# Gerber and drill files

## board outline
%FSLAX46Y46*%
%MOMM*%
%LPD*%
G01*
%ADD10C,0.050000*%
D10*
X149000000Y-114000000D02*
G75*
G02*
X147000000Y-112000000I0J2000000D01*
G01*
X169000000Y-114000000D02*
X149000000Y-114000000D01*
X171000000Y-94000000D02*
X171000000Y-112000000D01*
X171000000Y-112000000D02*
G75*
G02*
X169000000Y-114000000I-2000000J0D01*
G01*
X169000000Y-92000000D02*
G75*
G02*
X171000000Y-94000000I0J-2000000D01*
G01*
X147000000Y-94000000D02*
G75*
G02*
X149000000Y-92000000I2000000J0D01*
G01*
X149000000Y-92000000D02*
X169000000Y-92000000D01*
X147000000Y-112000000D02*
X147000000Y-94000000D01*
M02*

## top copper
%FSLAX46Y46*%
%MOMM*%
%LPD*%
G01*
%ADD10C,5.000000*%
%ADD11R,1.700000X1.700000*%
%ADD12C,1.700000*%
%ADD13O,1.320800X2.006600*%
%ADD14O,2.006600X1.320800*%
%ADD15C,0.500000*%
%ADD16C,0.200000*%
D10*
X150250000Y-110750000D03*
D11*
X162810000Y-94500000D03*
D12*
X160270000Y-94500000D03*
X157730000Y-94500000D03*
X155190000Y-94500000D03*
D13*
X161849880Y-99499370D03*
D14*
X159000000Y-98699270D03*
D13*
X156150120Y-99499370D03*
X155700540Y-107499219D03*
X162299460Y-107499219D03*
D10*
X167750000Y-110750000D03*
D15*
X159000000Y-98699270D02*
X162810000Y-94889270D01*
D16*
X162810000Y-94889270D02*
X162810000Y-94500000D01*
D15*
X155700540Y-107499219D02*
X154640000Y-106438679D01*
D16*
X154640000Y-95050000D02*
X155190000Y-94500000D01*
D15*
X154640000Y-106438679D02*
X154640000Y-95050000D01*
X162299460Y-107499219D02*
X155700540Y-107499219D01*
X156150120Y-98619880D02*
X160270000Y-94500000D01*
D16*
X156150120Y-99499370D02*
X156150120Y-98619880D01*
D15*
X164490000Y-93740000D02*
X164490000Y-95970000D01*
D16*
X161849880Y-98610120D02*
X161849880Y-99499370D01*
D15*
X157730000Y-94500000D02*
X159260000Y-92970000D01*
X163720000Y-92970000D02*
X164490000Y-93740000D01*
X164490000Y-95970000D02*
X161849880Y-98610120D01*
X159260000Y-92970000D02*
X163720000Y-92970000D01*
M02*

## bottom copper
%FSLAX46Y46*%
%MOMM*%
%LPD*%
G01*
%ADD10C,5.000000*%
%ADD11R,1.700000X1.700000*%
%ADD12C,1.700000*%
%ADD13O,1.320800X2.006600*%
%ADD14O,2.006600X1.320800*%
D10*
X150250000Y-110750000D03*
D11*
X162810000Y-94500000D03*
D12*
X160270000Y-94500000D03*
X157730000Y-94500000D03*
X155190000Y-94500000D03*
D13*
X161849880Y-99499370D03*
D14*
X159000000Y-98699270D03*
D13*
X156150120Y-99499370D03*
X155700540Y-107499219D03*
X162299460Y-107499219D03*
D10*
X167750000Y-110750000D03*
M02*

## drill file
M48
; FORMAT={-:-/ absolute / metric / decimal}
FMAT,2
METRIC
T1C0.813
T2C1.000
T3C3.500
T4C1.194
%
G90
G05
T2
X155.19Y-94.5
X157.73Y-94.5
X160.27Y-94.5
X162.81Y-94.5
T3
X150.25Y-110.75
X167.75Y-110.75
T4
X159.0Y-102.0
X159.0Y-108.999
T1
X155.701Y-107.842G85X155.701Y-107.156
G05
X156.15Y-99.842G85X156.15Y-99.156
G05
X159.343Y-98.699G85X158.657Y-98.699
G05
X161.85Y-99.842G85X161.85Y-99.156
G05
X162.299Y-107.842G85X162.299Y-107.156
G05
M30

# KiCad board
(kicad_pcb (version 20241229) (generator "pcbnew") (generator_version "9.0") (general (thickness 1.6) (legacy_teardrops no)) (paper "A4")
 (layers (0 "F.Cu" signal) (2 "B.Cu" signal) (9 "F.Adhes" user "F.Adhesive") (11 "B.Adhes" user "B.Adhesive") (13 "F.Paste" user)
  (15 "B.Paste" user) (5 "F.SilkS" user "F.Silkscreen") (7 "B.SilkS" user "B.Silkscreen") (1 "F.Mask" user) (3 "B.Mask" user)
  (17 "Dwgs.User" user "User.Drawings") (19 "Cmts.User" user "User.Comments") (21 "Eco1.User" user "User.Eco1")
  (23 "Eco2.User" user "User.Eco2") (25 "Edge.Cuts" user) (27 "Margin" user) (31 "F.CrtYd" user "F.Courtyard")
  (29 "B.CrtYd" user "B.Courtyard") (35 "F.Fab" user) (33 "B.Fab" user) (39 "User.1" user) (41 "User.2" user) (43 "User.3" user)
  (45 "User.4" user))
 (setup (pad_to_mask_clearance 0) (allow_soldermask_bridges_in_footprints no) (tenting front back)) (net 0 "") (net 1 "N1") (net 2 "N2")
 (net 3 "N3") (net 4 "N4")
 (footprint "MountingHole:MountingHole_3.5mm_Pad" (layer "F.Cu") (at 150.25 110.75)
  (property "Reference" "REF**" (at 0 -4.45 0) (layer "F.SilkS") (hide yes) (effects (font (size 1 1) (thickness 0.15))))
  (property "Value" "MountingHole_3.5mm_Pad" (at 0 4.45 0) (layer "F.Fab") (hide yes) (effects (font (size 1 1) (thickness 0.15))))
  (pad "" thru_hole circle (at 0 0) (size 5 5) (drill 3.5) (layers "*.Cu" "*.Mask") (remove_unused_layers no) (zone_connect 2)))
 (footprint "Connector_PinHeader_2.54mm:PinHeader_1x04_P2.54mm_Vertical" (layer "F.Cu") (at 162.81 94.5 -90)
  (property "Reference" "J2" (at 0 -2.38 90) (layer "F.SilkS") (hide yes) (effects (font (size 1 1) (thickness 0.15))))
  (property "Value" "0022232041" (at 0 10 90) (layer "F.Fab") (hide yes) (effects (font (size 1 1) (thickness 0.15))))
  (pad "1" thru_hole rect (at 0 0 270) (size 1.7 1.7) (drill 1) (layers "*.Cu" "*.Mask") (remove_unused_layers no) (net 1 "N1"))
  (pad "2" thru_hole circle (at 0 2.54 270) (size 1.7 1.7) (drill 1) (layers "*.Cu" "*.Mask") (remove_unused_layers no) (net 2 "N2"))
  (pad "3" thru_hole circle (at 0 5.08 270) (size 1.7 1.7) (drill 1) (layers "*.Cu" "*.Mask") (remove_unused_layers no) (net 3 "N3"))
  (pad "4" thru_hole circle (at 0 7.62 270) (size 1.7 1.7) (drill 1) (layers "*.Cu" "*.Mask") (remove_unused_layers no) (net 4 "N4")))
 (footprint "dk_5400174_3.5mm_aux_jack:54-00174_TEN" (layer "F.Cu") (at 159 106.78282)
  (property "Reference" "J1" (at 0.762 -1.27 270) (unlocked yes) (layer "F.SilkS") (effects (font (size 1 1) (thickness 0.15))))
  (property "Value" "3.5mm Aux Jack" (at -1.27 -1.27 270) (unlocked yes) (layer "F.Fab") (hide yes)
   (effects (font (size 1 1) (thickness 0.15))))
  (pad "" np_thru_hole circle (at 0 -4.78282 180) (size 1.1938 1.1938) (drill 1.1938) (layers "*.Cu" "*.Mask"))
  (pad "" np_thru_hole circle (at 0 2.21615 180) (size 1.1938 1.1938) (drill 1.1938) (layers "*.Cu" "*.Mask"))
  (pad "1" thru_hole oval (at 2.84988 -7.28345 180) (size 1.3208 2.0066) (drill oval 0.8128 1.4986) (layers "*.Cu" "*.Mask")
   (remove_unused_layers no) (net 3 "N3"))
  (pad "2" thru_hole oval (at 0 -8.08355 180) (size 2.0066 1.3208) (drill oval 1.4986 0.8128) (layers "*.Cu" "*.Mask")
   (remove_unused_layers no) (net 1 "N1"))
  (pad "3" thru_hole oval (at -2.84988 -7.28345 180) (size 1.3208 2.0066) (drill oval 0.8128 1.4986) (layers "*.Cu" "*.Mask")
   (remove_unused_layers no) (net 2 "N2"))
  (pad "4" thru_hole oval (at -3.29946 0.716399 180) (size 1.3208 2.0066) (drill oval 0.8128 1.4986) (layers "*.Cu" "*.Mask")
   (remove_unused_layers no) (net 4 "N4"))
  (pad "4" thru_hole oval (at 3.29946 0.716399 180) (size 1.3208 2.0066) (drill oval 0.8128 1.4986) (layers "*.Cu" "*.Mask")
   (remove_unused_layers no) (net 4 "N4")))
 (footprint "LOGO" (layer "F.Cu") (at 167 101.5 -90)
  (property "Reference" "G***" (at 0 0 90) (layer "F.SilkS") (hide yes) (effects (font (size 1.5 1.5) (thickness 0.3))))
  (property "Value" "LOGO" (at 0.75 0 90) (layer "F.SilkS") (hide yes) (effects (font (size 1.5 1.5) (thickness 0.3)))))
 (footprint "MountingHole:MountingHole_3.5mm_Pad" (layer "F.Cu") (at 167.75 110.75)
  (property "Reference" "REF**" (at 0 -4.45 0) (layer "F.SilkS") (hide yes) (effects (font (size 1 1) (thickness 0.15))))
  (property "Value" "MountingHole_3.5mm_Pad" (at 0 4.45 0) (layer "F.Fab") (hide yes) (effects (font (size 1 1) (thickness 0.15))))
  (pad "" thru_hole circle (at 0 0) (size 5 5) (drill 3.5) (layers "*.Cu" "*.Mask") (remove_unused_layers no) (zone_connect 2)))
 (gr_arc (start 149 114) (mid 147.585786 113.414214) (end 147 112) (stroke (width 0.05) (type default)) (layer "Edge.Cuts"))
 (gr_line (start 169 114) (end 149 114) (stroke (width 0.05) (type default)) (layer "Edge.Cuts"))
 (gr_line (start 171 94) (end 171 112) (stroke (width 0.05) (type default)) (layer "Edge.Cuts"))
 (gr_arc (start 171 112) (mid 170.414214 113.414214) (end 169 114) (stroke (width 0.05) (type default)) (layer "Edge.Cuts"))
 (gr_arc (start 169 92) (mid 170.414214 92.585786) (end 171 94) (stroke (width 0.05) (type default)) (layer "Edge.Cuts"))
 (gr_arc (start 147 94) (mid 147.585786 92.585786) (end 149 92) (stroke (width 0.05) (type default)) (layer "Edge.Cuts"))
 (gr_line (start 149 92) (end 169 92) (stroke (width 0.05) (type default)) (layer "Edge.Cuts"))
 (gr_line (start 147 112) (end 147 94) (stroke (width 0.05) (type default)) (layer "Edge.Cuts"))
 (segment (start 159 98.69927) (end 162.81 94.88927) (width 0.5) (layer "F.Cu") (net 1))
 (segment (start 162.81 94.88927) (end 162.81 94.5) (width 0.2) (layer "F.Cu") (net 1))
 (segment (start 155.70054 107.499219) (end 154.64 106.438679) (width 0.5) (layer "F.Cu") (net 4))
 (segment (start 154.64 95.05) (end 155.19 94.5) (width 0.2) (layer "F.Cu") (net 4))
 (segment (start 154.64 106.438679) (end 154.64 95.05) (width 0.5) (layer "F.Cu") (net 4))
 (segment (start 162.29946 107.499219) (end 155.70054 107.499219) (width 0.5) (layer "F.Cu") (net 4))
 (segment (start 156.15012 98.61988) (end 160.27 94.5) (width 0.5) (layer "F.Cu") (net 2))
 (segment (start 156.15012 99.49937) (end 156.15012 98.61988) (width 0.2) (layer "F.Cu") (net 2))
 (segment (start 164.49 93.74) (end 164.49 95.97) (width 0.5) (layer "F.Cu") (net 3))
 (segment (start 161.84988 98.61012) (end 161.84988 99.49937) (width 0.2) (layer "F.Cu") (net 3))
 (segment (start 157.73 94.5) (end 159.26 92.97) (width 0.5) (layer "F.Cu") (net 3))
 (segment (start 163.72 92.97) (end 164.49 93.74) (width 0.5) (layer "F.Cu") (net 3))
 (segment (start 164.49 95.97) (end 161.84988 98.61012) (width 0.5) (layer "F.Cu") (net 3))
 (segment (start 159.26 92.97) (end 163.72 92.97) (width 0.5) (layer "F.Cu") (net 3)))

